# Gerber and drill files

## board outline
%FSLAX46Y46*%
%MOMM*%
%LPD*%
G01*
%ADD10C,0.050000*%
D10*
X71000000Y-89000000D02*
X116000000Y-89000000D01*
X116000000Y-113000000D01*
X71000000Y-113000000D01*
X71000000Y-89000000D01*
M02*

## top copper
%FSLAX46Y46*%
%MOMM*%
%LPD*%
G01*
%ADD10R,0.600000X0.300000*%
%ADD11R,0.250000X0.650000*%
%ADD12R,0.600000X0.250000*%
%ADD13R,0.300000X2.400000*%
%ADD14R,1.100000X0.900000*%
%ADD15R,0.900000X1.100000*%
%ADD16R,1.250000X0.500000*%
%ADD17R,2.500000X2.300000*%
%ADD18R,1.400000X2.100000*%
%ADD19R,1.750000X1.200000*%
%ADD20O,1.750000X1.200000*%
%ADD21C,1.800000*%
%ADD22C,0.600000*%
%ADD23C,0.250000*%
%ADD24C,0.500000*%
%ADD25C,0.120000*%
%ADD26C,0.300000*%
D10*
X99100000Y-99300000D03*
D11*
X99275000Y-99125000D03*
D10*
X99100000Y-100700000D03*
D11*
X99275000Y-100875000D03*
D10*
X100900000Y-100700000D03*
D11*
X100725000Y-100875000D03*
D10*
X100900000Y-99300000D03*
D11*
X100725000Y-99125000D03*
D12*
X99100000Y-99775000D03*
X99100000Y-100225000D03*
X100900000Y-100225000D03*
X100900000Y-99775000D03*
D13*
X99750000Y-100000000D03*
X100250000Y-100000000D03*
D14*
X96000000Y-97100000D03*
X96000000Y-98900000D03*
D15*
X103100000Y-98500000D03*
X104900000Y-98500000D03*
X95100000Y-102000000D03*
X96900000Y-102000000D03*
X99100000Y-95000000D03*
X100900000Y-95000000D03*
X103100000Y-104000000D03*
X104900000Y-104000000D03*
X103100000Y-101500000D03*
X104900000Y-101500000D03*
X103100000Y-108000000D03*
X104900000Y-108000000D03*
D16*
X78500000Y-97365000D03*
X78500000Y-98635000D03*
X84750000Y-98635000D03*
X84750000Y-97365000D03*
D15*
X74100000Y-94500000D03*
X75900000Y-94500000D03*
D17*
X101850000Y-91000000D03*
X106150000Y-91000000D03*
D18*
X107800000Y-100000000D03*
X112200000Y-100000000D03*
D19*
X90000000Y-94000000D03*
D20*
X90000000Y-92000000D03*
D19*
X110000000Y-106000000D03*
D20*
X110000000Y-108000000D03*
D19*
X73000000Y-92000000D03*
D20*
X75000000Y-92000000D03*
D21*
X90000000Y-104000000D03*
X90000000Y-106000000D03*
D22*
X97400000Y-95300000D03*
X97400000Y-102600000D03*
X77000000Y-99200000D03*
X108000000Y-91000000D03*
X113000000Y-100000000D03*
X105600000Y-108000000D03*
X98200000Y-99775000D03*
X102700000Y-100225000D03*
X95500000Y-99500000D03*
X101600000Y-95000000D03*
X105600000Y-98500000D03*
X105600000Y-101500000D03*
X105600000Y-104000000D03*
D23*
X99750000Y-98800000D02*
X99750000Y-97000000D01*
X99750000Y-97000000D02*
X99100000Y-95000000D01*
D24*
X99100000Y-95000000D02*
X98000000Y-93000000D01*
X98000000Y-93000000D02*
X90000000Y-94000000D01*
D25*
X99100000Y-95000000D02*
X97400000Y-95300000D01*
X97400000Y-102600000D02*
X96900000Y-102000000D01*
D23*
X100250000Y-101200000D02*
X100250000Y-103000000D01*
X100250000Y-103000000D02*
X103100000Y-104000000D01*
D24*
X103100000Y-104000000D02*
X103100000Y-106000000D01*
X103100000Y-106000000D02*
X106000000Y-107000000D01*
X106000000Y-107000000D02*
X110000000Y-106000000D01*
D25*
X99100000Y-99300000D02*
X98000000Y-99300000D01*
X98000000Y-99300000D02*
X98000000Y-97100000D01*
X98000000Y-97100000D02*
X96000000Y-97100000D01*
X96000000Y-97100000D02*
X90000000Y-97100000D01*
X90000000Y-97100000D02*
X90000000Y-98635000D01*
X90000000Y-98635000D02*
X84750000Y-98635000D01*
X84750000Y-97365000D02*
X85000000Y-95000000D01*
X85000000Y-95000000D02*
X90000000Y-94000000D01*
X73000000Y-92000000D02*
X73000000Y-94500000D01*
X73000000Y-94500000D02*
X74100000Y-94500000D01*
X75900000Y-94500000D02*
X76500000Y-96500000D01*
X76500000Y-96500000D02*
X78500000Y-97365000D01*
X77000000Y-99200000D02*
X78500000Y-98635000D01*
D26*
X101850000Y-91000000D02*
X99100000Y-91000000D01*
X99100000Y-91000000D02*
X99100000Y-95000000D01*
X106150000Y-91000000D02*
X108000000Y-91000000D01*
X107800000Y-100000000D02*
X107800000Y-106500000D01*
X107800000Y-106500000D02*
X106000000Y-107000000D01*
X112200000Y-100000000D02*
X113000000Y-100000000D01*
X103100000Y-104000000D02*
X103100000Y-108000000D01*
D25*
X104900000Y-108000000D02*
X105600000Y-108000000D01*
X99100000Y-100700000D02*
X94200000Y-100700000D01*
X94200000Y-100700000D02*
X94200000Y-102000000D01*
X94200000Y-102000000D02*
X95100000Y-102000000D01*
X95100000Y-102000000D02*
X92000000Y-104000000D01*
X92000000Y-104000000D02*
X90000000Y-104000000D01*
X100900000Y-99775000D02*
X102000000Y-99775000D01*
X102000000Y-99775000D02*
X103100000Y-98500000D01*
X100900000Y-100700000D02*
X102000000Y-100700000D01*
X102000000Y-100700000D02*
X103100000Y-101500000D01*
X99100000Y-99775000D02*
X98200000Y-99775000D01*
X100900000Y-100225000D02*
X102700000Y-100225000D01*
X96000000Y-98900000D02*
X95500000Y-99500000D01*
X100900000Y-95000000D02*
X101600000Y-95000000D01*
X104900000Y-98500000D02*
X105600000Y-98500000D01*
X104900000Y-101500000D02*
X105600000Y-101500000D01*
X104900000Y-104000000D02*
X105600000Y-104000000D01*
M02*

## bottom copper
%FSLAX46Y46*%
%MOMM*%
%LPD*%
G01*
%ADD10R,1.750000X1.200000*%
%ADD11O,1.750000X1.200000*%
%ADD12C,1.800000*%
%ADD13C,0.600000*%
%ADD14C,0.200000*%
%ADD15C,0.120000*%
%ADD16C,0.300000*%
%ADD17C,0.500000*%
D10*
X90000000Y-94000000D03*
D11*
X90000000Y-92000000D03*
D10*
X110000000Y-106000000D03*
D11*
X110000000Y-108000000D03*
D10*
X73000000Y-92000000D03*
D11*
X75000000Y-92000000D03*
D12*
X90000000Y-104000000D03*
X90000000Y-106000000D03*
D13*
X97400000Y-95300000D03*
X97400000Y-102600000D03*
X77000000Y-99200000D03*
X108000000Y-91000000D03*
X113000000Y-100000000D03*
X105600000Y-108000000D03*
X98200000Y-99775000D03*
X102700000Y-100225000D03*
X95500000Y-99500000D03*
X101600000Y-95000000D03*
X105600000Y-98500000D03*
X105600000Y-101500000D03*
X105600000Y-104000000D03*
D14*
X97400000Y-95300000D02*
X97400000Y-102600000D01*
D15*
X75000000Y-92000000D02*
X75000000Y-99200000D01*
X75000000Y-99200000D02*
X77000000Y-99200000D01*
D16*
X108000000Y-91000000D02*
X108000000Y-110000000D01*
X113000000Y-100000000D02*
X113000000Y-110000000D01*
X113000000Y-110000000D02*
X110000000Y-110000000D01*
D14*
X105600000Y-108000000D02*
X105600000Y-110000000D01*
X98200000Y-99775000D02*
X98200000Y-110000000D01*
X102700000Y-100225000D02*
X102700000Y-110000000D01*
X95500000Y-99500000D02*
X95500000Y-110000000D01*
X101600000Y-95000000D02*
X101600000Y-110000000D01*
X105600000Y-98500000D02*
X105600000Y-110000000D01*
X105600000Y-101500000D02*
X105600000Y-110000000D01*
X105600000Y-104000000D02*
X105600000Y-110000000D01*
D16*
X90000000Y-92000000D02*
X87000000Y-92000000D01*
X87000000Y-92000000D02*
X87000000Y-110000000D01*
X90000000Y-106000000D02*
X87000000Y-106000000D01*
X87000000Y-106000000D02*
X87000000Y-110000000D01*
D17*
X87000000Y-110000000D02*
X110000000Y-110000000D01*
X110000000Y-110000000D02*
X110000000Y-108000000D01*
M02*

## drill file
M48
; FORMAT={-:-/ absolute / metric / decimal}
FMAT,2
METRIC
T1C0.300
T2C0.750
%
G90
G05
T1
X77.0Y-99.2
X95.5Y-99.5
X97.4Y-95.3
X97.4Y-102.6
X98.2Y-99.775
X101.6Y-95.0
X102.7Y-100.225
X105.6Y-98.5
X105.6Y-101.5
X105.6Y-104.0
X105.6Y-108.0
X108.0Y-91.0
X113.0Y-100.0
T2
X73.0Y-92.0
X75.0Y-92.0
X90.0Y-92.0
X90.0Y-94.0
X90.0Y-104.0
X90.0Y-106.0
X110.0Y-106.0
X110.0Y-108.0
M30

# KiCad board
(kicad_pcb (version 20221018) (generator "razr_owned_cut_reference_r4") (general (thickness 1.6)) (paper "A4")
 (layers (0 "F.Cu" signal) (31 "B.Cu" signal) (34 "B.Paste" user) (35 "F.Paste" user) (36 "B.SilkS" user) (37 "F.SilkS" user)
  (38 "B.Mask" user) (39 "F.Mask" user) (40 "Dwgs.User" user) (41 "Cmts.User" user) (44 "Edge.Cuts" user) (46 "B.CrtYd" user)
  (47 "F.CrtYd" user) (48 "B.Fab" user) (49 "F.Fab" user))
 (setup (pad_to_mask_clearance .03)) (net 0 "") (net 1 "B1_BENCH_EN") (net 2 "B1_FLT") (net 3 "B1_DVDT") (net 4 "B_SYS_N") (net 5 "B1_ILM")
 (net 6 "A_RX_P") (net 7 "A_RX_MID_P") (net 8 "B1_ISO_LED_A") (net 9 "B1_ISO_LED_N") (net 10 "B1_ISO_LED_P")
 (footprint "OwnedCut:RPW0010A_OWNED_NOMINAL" (layer "F.Cu") (at 100 100)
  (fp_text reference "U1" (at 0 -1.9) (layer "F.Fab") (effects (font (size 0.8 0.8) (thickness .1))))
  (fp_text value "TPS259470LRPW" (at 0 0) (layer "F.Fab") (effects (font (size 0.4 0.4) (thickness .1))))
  (pad "1" smd rect (at -0.9 -0.7) (size 0.6 0.3) (layers "F.Cu" "F.Paste" "F.Mask") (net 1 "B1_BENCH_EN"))
  (pad "1" smd rect (at -0.725 -0.875) (size 0.25 0.65) (layers "F.Cu" "F.Paste" "F.Mask") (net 1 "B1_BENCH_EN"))
  (pad "4" smd rect (at -0.9 0.7) (size 0.6 0.3) (layers "F.Cu" "F.Paste" "F.Mask") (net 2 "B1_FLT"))
  (pad "4" smd rect (at -0.725 0.875) (size 0.25 0.65) (layers "F.Cu" "F.Paste" "F.Mask") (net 2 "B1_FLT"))
  (pad "7" smd rect (at 0.9 0.7) (size 0.6 0.3) (layers "F.Cu" "F.Paste" "F.Mask") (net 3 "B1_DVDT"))
  (pad "7" smd rect (at 0.725 0.875) (size 0.25 0.65) (layers "F.Cu" "F.Paste" "F.Mask") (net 3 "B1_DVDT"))
  (pad "10" smd rect (at 0.9 -0.7) (size 0.6 0.3) (layers "F.Cu" "F.Paste" "F.Mask"))
  (pad "10" smd rect (at 0.725 -0.875) (size 0.25 0.65) (layers "F.Cu" "F.Paste" "F.Mask"))
  (pad "2" smd rect (at -0.9 -0.225) (size 0.6 0.25) (layers "F.Cu" "F.Paste" "F.Mask") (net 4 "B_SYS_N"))
  (pad "3" smd rect (at -0.9 0.225) (size 0.6 0.25) (layers "F.Cu" "F.Paste" "F.Mask"))
  (pad "8" smd rect (at 0.9 0.225) (size 0.6 0.25) (layers "F.Cu" "F.Paste" "F.Mask") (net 4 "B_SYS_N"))
  (pad "9" smd rect (at 0.9 -0.225) (size 0.6 0.25) (layers "F.Cu" "F.Paste" "F.Mask") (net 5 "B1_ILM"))
  (pad "5" smd rect (at -0.25 0) (size 0.3 2.4) (layers "F.Cu" "F.Paste" "F.Mask") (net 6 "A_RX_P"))
  (pad "6" smd rect (at 0.25 0) (size 0.3 2.4) (layers "F.Cu" "F.Paste" "F.Mask") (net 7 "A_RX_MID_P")))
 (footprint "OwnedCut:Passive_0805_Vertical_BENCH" (layer "F.Cu") (at 96 98)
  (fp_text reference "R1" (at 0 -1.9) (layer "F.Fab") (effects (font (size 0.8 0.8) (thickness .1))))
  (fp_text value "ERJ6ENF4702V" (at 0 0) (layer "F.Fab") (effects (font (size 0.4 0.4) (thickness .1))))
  (pad "1" smd rect (at 0 -0.9) (size 1.1 0.9) (layers "F.Cu" "F.Paste" "F.Mask") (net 1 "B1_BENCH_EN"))
  (pad "2" smd rect (at 0 0.9) (size 1.1 0.9) (layers "F.Cu" "F.Paste" "F.Mask") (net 4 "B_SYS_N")))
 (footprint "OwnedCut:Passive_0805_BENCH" (layer "F.Cu") (at 104 98.5)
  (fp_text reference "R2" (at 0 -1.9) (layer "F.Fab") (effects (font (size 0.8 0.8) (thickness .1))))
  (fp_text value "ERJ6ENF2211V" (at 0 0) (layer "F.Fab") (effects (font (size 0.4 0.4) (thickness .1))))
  (pad "1" smd rect (at -0.9 0) (size 0.9 1.1) (layers "F.Cu" "F.Paste" "F.Mask") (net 5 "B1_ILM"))
  (pad "2" smd rect (at 0.9 0) (size 0.9 1.1) (layers "F.Cu" "F.Paste" "F.Mask") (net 4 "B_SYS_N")))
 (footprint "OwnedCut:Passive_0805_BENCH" (layer "F.Cu") (at 96 102)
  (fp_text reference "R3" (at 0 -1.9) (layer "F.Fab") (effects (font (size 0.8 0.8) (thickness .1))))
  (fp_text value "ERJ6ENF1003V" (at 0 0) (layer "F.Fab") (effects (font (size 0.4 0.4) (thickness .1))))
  (pad "1" smd rect (at -0.9 0) (size 0.9 1.1) (layers "F.Cu" "F.Paste" "F.Mask") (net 2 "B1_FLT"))
  (pad "2" smd rect (at 0.9 0) (size 0.9 1.1) (layers "F.Cu" "F.Paste" "F.Mask") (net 6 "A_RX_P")))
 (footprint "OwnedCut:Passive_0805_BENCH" (layer "F.Cu") (at 100 95)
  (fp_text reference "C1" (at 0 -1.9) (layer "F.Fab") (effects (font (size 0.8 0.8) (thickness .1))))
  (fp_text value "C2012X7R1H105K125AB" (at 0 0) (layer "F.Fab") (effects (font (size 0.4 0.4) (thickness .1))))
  (pad "1" smd rect (at -0.9 0) (size 0.9 1.1) (layers "F.Cu" "F.Paste" "F.Mask") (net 6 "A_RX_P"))
  (pad "2" smd rect (at 0.9 0) (size 0.9 1.1) (layers "F.Cu" "F.Paste" "F.Mask") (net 4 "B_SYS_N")))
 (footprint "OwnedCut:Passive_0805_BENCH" (layer "F.Cu") (at 104 104)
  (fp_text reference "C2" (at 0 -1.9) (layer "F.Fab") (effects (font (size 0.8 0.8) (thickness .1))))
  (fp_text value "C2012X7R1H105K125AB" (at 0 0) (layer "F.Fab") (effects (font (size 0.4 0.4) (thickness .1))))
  (pad "1" smd rect (at -0.9 0) (size 0.9 1.1) (layers "F.Cu" "F.Paste" "F.Mask") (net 7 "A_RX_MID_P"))
  (pad "2" smd rect (at 0.9 0) (size 0.9 1.1) (layers "F.Cu" "F.Paste" "F.Mask") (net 4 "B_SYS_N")))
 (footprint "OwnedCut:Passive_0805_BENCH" (layer "F.Cu") (at 104 101.5)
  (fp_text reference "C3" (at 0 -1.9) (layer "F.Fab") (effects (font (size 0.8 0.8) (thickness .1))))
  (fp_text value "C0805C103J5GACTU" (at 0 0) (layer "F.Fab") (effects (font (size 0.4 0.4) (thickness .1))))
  (pad "1" smd rect (at -0.9 0) (size 0.9 1.1) (layers "F.Cu" "F.Paste" "F.Mask") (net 3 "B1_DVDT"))
  (pad "2" smd rect (at 0.9 0) (size 0.9 1.1) (layers "F.Cu" "F.Paste" "F.Mask") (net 4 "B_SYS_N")))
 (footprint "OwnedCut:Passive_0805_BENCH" (layer "F.Cu") (at 104 108)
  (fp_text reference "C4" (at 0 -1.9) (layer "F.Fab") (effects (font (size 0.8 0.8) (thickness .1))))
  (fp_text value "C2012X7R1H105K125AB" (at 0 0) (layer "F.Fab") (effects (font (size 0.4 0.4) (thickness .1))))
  (pad "1" smd rect (at -0.9 0) (size 0.9 1.1) (layers "F.Cu" "F.Paste" "F.Mask") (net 7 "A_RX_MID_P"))
  (pad "2" smd rect (at 0.9 0) (size 0.9 1.1) (layers "F.Cu" "F.Paste" "F.Mask") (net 4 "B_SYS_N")))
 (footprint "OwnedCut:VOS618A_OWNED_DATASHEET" (layer "F.Cu") (at 81.625 98)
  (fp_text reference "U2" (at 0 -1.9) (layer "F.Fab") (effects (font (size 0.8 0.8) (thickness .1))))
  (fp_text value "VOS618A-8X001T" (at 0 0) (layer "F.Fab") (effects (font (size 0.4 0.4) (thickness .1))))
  (pad "1" smd rect (at -3.125 -0.635) (size 1.25 0.5) (layers "F.Cu" "F.Paste" "F.Mask") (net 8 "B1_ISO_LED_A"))
  (pad "2" smd rect (at -3.125 0.635) (size 1.25 0.5) (layers "F.Cu" "F.Paste" "F.Mask") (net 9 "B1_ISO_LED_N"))
  (pad "3" smd rect (at 3.125 0.635) (size 1.25 0.5) (layers "F.Cu" "F.Paste" "F.Mask") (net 1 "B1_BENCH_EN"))
  (pad "4" smd rect (at 3.125 -0.635) (size 1.25 0.5) (layers "F.Cu" "F.Paste" "F.Mask") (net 6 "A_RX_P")))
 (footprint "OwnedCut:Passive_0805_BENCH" (layer "F.Cu") (at 75 94.5)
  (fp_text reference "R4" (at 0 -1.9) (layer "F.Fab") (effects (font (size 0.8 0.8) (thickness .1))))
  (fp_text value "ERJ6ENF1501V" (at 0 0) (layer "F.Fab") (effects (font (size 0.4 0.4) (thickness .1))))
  (pad "1" smd rect (at -0.9 0) (size 0.9 1.1) (layers "F.Cu" "F.Paste" "F.Mask") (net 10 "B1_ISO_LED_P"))
  (pad "2" smd rect (at 0.9 0) (size 0.9 1.1) (layers "F.Cu" "F.Paste" "F.Mask") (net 8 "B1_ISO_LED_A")))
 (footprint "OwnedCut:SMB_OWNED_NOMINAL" (layer "F.Cu") (at 104 91)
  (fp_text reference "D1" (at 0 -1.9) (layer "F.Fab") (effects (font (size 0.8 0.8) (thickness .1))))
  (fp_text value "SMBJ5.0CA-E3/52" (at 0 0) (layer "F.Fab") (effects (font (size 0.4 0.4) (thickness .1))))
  (pad "1" smd rect (at -2.15 0) (size 2.5 2.3) (layers "F.Cu" "F.Paste" "F.Mask") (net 6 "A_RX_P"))
  (pad "2" smd rect (at 2.15 0) (size 2.5 2.3) (layers "F.Cu" "F.Paste" "F.Mask") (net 4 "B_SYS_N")))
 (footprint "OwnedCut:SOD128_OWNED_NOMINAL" (layer "F.Cu") (at 110 100)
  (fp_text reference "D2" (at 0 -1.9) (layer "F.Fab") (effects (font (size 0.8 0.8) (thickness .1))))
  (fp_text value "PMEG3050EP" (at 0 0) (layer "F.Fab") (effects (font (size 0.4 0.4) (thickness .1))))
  (pad "1" smd rect (at -2.2 0) (size 1.4 2.1) (layers "F.Cu" "F.Paste" "F.Mask") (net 7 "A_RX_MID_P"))
  (pad "2" smd rect (at 2.2 0) (size 1.4 2.1) (layers "F.Cu" "F.Paste" "F.Mask") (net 4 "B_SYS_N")))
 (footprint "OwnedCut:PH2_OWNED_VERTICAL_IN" (layer "F.Cu") (at 90 94)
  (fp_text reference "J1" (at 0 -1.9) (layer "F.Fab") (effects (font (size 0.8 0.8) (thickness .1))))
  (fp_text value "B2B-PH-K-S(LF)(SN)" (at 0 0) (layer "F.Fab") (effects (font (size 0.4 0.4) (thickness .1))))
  (pad "1" thru_hole rect (at 0 0) (size 1.75 1.2) (drill .75) (layers "*.Cu" "*.Mask") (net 6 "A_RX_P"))
  (pad "2" thru_hole oval (at 0 -2) (size 1.75 1.2) (drill .75) (layers "*.Cu" "*.Mask") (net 4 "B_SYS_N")))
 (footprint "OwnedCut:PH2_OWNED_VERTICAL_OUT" (layer "F.Cu") (at 110 106)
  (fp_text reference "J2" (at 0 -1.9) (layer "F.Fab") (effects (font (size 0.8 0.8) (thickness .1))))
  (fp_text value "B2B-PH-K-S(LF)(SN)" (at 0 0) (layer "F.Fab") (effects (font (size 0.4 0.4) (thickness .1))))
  (pad "1" thru_hole rect (at 0 0) (size 1.75 1.2) (drill .75) (layers "*.Cu" "*.Mask") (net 7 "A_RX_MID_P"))
  (pad "2" thru_hole oval (at 0 2) (size 1.75 1.2) (drill .75) (layers "*.Cu" "*.Mask") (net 4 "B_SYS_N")))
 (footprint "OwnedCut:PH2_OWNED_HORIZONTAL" (layer "F.Cu") (at 73 92)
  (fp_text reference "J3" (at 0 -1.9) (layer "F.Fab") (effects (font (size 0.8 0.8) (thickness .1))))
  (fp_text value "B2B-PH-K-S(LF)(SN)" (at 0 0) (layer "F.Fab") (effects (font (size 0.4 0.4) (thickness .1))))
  (pad "1" thru_hole rect (at 0 0) (size 1.75 1.2) (drill .75) (layers "*.Cu" "*.Mask") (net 10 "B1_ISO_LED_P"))
  (pad "2" thru_hole oval (at 2 0) (size 1.75 1.2) (drill .75) (layers "*.Cu" "*.Mask") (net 9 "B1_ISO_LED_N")))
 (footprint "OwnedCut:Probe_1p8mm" (layer "F.Cu") (at 90 104)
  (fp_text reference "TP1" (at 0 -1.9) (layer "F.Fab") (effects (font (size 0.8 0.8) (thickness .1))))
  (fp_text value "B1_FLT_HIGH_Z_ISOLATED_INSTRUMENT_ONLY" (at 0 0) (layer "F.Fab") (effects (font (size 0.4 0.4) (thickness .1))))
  (pad "1" thru_hole circle (at 0 0) (size 1.8 1.8) (drill .75) (layers "*.Cu" "*.Mask") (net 2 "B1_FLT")))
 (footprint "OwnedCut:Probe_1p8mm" (layer "F.Cu") (at 90 106)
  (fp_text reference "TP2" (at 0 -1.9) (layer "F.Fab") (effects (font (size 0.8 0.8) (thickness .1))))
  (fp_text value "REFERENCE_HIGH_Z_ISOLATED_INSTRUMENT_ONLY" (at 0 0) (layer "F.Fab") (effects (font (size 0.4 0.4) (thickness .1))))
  (pad "1" thru_hole circle (at 0 0) (size 1.8 1.8) (drill .75) (layers "*.Cu" "*.Mask") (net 4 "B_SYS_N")))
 (segment (start 99.75 98.8) (end 99.75 97) (width 0.25) (layer "F.Cu") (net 6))
 (segment (start 99.75 97) (end 99.1 95) (width 0.25) (layer "F.Cu") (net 6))
 (segment (start 99.1 95) (end 98 93) (width 0.5) (layer "F.Cu") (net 6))
 (segment (start 98 93) (end 90 94) (width 0.5) (layer "F.Cu") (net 6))
 (segment (start 99.1 95) (end 97.4 95.3) (width 0.12) (layer "F.Cu") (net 6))
 (via (at 97.4 95.3) (size .6) (drill .3) (layers "F.Cu" "B.Cu") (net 6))
 (segment (start 97.4 95.3) (end 97.4 102.6) (width 0.2) (layer "B.Cu") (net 6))
 (via (at 97.4 102.6) (size .6) (drill .3) (layers "F.Cu" "B.Cu") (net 6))
 (segment (start 97.4 102.6) (end 96.9 102) (width 0.12) (layer "F.Cu") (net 6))
 (segment (start 100.25 101.2) (end 100.25 103) (width 0.25) (layer "F.Cu") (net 7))
 (segment (start 100.25 103) (end 103.1 104) (width 0.25) (layer "F.Cu") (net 7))
 (segment (start 103.1 104) (end 103.1 106) (width 0.5) (layer "F.Cu") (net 7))
 (segment (start 103.1 106) (end 106 107) (width 0.5) (layer "F.Cu") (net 7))
 (segment (start 106 107) (end 110 106) (width 0.5) (layer "F.Cu") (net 7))
 (segment (start 99.1 99.3) (end 98 99.3) (width 0.12) (layer "F.Cu") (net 1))
 (segment (start 98 99.3) (end 98 97.1) (width 0.12) (layer "F.Cu") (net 1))
 (segment (start 98 97.1) (end 96 97.1) (width 0.12) (layer "F.Cu") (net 1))
 (segment (start 96 97.1) (end 90 97.1) (width 0.12) (layer "F.Cu") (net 1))
 (segment (start 90 97.1) (end 90 98.635) (width 0.12) (layer "F.Cu") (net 1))
 (segment (start 90 98.635) (end 84.75 98.635) (width 0.12) (layer "F.Cu") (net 1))
 (segment (start 84.75 97.365) (end 85 95) (width 0.12) (layer "F.Cu") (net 6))
 (segment (start 85 95) (end 90 94) (width 0.12) (layer "F.Cu") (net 6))
 (segment (start 73 92) (end 73 94.5) (width 0.12) (layer "F.Cu") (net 10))
 (segment (start 73 94.5) (end 74.1 94.5) (width 0.12) (layer "F.Cu") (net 10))
 (segment (start 75.9 94.5) (end 76.5 96.5) (width 0.12) (layer "F.Cu") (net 8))
 (segment (start 76.5 96.5) (end 78.5 97.365) (width 0.12) (layer "F.Cu") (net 8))
 (segment (start 75 92) (end 75 99.2) (width 0.12) (layer "B.Cu") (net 9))
 (segment (start 75 99.2) (end 77 99.2) (width 0.12) (layer "B.Cu") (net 9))
 (via (at 77 99.2) (size .6) (drill .3) (layers "F.Cu" "B.Cu") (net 9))
 (segment (start 77 99.2) (end 78.5 98.635) (width 0.12) (layer "F.Cu") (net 9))
 (segment (start 101.85 91) (end 99.1 91) (width 0.3) (layer "F.Cu") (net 6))
 (segment (start 99.1 91) (end 99.1 95) (width 0.3) (layer "F.Cu") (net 6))
 (segment (start 106.15 91) (end 108 91) (width 0.3) (layer "F.Cu") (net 4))
 (via (at 108 91) (size .6) (drill .3) (layers "F.Cu" "B.Cu") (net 4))
 (segment (start 108 91) (end 108 110) (width 0.3) (layer "B.Cu") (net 4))
 (segment (start 107.8 100) (end 107.8 106.5) (width 0.3) (layer "F.Cu") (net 7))
 (segment (start 107.8 106.5) (end 106 107) (width 0.3) (layer "F.Cu") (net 7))
 (segment (start 112.2 100) (end 113 100) (width 0.3) (layer "F.Cu") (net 4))
 (via (at 113 100) (size .6) (drill .3) (layers "F.Cu" "B.Cu") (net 4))
 (segment (start 113 100) (end 113 110) (width 0.3) (layer "B.Cu") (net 4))
 (segment (start 113 110) (end 110 110) (width 0.3) (layer "B.Cu") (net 4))
 (segment (start 103.1 104) (end 103.1 108) (width 0.3) (layer "F.Cu") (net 7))
 (segment (start 104.9 108) (end 105.6 108) (width 0.12) (layer "F.Cu") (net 4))
 (via (at 105.6 108) (size .6) (drill .3) (layers "F.Cu" "B.Cu") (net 4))
 (segment (start 105.6 108) (end 105.6 110) (width 0.2) (layer "B.Cu") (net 4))
 (segment (start 99.1 100.7) (end 94.2 100.7) (width 0.12) (layer "F.Cu") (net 2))
 (segment (start 94.2 100.7) (end 94.2 102) (width 0.12) (layer "F.Cu") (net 2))
 (segment (start 94.2 102) (end 95.1 102) (width 0.12) (layer "F.Cu") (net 2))
 (segment (start 95.1 102) (end 92 104) (width 0.12) (layer "F.Cu") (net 2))
 (segment (start 92 104) (end 90 104) (width 0.12) (layer "F.Cu") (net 2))
 (segment (start 100.9 99.775) (end 102 99.775) (width 0.12) (layer "F.Cu") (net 5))
 (segment (start 102 99.775) (end 103.1 98.5) (width 0.12) (layer "F.Cu") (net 5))
 (segment (start 100.9 100.7) (end 102 100.7) (width 0.12) (layer "F.Cu") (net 3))
 (segment (start 102 100.7) (end 103.1 101.5) (width 0.12) (layer "F.Cu") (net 3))
 (segment (start 99.1 99.775) (end 98.2 99.775) (width 0.12) (layer "F.Cu") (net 4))
 (via (at 98.2 99.775) (size .6) (drill .3) (layers "F.Cu" "B.Cu") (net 4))
 (segment (start 98.2 99.775) (end 98.2 110) (width 0.2) (layer "B.Cu") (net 4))
 (segment (start 100.9 100.225) (end 102.7 100.225) (width 0.12) (layer "F.Cu") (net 4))
 (via (at 102.7 100.225) (size .6) (drill .3) (layers "F.Cu" "B.Cu") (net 4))
 (segment (start 102.7 100.225) (end 102.7 110) (width 0.2) (layer "B.Cu") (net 4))
 (segment (start 96 98.9) (end 95.5 99.5) (width 0.12) (layer "F.Cu") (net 4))
 (via (at 95.5 99.5) (size .6) (drill .3) (layers "F.Cu" "B.Cu") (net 4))
 (segment (start 95.5 99.5) (end 95.5 110) (width 0.2) (layer "B.Cu") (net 4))
 (segment (start 100.9 95) (end 101.6 95) (width 0.12) (layer "F.Cu") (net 4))
 (via (at 101.6 95) (size .6) (drill .3) (layers "F.Cu" "B.Cu") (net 4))
 (segment (start 101.6 95) (end 101.6 110) (width 0.2) (layer "B.Cu") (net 4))
 (segment (start 104.9 98.5) (end 105.6 98.5) (width 0.12) (layer "F.Cu") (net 4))
 (via (at 105.6 98.5) (size .6) (drill .3) (layers "F.Cu" "B.Cu") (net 4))
 (segment (start 105.6 98.5) (end 105.6 110) (width 0.2) (layer "B.Cu") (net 4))
 (segment (start 104.9 101.5) (end 105.6 101.5) (width 0.12) (layer "F.Cu") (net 4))
 (via (at 105.6 101.5) (size .6) (drill .3) (layers "F.Cu" "B.Cu") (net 4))
 (segment (start 105.6 101.5) (end 105.6 110) (width 0.2) (layer "B.Cu") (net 4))
 (segment (start 104.9 104) (end 105.6 104) (width 0.12) (layer "F.Cu") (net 4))
 (via (at 105.6 104) (size .6) (drill .3) (layers "F.Cu" "B.Cu") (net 4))
 (segment (start 105.6 104) (end 105.6 110) (width 0.2) (layer "B.Cu") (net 4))
 (segment (start 90 92) (end 87 92) (width 0.3) (layer "B.Cu") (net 4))
 (segment (start 87 92) (end 87 110) (width 0.3) (layer "B.Cu") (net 4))
 (segment (start 90 106) (end 87 106) (width 0.3) (layer "B.Cu") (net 4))
 (segment (start 87 106) (end 87 110) (width 0.3) (layer "B.Cu") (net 4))
 (segment (start 87 110) (end 110 110) (width 0.5) (layer "B.Cu") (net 4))
 (segment (start 110 110) (end 110 108) (width 0.5) (layer "B.Cu") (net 4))
 (gr_rect (start 71 89) (end 116 113) (stroke (width .05) (type default)) (fill none) (layer "Edge.Cuts")))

